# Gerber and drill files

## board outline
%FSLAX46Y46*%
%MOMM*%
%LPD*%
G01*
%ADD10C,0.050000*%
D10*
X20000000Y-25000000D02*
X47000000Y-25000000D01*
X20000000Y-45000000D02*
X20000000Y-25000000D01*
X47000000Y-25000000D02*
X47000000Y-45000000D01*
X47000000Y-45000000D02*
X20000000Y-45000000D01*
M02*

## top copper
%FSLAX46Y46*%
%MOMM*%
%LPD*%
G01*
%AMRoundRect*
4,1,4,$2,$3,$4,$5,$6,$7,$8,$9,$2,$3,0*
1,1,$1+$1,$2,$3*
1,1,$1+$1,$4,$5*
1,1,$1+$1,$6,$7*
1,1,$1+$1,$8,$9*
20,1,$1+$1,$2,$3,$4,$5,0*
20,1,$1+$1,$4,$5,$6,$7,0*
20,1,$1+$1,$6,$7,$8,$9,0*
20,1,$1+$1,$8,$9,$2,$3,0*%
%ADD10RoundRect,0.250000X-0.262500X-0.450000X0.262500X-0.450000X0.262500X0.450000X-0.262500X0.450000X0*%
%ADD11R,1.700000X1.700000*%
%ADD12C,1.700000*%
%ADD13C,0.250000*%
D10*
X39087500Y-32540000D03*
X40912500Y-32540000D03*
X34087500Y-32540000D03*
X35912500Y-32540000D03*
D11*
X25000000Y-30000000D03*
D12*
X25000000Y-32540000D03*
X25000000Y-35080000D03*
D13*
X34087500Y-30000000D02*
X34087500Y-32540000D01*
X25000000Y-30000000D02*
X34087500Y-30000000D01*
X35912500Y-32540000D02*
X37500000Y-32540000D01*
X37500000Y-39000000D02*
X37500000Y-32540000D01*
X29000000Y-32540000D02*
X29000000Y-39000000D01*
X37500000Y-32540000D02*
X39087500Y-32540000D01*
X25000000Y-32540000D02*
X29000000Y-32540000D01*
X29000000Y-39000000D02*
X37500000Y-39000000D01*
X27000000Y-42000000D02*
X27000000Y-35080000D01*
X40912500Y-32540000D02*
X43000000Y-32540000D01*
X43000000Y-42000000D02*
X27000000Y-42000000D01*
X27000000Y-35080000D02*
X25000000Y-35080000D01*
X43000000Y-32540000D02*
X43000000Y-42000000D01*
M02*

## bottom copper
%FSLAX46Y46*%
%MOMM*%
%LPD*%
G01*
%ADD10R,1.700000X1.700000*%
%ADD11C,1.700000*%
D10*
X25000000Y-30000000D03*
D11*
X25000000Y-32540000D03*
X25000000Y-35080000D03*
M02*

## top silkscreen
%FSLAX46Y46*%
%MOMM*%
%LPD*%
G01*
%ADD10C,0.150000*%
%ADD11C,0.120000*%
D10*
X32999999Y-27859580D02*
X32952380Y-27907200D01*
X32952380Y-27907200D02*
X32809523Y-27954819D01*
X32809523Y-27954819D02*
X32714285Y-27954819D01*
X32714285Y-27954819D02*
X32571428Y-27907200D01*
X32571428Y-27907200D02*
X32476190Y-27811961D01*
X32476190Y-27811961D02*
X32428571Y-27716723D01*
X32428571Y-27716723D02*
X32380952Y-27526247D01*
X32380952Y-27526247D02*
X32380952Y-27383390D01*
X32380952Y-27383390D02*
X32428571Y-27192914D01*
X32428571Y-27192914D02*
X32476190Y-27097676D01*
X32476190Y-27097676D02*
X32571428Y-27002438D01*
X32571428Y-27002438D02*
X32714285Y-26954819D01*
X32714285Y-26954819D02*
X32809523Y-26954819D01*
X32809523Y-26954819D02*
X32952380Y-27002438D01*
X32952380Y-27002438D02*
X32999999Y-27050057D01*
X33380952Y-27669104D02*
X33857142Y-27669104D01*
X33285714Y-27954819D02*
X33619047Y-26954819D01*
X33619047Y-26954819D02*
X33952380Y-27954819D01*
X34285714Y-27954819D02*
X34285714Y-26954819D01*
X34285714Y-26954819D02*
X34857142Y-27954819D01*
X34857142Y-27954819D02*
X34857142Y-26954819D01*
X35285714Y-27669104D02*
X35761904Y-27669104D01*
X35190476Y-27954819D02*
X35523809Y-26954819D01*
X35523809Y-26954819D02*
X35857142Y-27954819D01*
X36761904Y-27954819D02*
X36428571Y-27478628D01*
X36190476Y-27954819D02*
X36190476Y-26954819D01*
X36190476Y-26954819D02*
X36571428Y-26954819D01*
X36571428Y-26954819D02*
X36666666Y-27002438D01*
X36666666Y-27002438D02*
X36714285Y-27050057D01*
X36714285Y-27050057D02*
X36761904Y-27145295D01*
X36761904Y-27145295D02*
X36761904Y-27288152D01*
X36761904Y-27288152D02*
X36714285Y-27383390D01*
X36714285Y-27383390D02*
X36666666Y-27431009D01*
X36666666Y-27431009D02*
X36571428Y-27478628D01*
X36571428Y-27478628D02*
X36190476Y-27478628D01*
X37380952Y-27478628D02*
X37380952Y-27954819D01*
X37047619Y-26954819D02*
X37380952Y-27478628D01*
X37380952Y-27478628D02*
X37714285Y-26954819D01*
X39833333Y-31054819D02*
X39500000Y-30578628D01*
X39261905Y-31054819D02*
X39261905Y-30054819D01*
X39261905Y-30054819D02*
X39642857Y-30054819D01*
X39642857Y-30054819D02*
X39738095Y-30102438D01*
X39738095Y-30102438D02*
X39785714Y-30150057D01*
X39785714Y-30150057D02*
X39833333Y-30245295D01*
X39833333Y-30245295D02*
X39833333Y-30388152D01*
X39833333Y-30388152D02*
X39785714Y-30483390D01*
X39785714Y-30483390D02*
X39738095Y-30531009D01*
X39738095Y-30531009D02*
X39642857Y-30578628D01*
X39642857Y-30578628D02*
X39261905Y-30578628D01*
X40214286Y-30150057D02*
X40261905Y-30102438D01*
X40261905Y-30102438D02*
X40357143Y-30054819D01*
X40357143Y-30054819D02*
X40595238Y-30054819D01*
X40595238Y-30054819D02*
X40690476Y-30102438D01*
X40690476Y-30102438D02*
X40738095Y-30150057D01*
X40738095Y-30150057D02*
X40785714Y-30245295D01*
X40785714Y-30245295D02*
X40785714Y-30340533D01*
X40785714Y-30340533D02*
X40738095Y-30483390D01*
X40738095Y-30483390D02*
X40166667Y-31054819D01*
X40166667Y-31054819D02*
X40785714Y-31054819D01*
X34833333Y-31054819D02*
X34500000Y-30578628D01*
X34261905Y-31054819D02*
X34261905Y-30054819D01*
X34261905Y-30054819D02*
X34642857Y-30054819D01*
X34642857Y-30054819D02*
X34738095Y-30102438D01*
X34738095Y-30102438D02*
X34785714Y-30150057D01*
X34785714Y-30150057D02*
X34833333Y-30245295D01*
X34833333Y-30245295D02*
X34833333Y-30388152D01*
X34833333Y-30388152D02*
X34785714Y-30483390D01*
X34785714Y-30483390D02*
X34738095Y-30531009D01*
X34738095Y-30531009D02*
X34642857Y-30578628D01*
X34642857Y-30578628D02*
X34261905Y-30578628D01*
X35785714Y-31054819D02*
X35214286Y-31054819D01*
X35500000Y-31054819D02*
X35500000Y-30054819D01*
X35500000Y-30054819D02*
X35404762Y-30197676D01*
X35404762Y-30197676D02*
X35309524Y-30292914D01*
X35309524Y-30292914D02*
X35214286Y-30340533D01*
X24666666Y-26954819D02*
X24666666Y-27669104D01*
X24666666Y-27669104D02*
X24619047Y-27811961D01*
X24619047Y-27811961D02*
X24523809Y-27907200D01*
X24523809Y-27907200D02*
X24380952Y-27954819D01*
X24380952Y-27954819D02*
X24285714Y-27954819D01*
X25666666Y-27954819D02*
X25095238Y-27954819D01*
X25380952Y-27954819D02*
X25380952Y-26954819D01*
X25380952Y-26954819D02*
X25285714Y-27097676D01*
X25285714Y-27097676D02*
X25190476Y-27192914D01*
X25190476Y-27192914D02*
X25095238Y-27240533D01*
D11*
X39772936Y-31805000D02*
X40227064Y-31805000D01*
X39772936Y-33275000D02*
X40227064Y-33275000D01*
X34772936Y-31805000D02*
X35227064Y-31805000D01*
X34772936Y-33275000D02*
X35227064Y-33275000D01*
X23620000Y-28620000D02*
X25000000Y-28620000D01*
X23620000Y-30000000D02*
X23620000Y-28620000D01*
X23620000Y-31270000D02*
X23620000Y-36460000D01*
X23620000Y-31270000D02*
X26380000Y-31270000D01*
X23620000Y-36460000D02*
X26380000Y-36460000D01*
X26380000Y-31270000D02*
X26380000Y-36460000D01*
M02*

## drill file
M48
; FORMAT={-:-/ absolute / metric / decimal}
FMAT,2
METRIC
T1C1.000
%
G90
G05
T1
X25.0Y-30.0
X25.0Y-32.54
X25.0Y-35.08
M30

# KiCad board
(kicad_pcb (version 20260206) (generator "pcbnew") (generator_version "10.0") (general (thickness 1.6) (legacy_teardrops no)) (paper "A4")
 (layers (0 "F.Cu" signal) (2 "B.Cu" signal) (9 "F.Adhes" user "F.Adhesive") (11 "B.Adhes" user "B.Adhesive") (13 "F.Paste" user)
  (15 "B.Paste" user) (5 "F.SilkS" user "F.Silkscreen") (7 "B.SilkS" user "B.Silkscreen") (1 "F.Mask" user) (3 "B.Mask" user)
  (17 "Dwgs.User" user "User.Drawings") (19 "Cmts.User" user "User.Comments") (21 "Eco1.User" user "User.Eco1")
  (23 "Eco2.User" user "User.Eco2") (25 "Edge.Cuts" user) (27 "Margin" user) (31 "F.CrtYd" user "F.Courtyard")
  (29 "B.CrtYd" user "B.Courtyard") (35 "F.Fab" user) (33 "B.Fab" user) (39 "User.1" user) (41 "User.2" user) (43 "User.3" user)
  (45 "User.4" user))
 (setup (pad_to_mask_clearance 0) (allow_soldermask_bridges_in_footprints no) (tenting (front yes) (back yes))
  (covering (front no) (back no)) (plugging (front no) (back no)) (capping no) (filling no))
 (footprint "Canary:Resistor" (layer "F.Cu") (at 40 32.54)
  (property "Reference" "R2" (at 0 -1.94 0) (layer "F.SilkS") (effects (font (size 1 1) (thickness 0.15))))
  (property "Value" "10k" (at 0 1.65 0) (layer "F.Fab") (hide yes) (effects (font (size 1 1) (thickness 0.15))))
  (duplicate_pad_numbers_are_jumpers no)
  (fp_line (start -0.227064 -0.735) (end 0.227064 -0.735) (stroke (width 0.12) (type solid)) (layer "F.SilkS"))
  (fp_line (start -0.227064 0.735) (end 0.227064 0.735) (stroke (width 0.12) (type solid)) (layer "F.SilkS"))
  (pad "1" smd roundrect (at -0.9125 0) (size 1.025 1.4) (layers "F.Cu" "F.Mask" "F.Paste") (roundrect_rratio 0.243902) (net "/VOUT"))
  (pad "2" smd roundrect (at 0.9125 0) (size 1.025 1.4) (layers "F.Cu" "F.Mask" "F.Paste") (roundrect_rratio 0.243902) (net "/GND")))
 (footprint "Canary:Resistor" (layer "F.Cu") (at 35 32.54)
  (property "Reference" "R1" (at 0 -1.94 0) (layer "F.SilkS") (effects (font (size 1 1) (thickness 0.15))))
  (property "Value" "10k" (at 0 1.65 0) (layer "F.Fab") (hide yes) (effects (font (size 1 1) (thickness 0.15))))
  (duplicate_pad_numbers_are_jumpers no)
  (fp_line (start -0.227064 -0.735) (end 0.227064 -0.735) (stroke (width 0.12) (type solid)) (layer "F.SilkS"))
  (fp_line (start -0.227064 0.735) (end 0.227064 0.735) (stroke (width 0.12) (type solid)) (layer "F.SilkS"))
  (pad "1" smd roundrect (at -0.9125 0) (size 1.025 1.4) (layers "F.Cu" "F.Mask" "F.Paste") (roundrect_rratio 0.243902) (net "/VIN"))
  (pad "2" smd roundrect (at 0.9125 0) (size 1.025 1.4) (layers "F.Cu" "F.Mask" "F.Paste") (roundrect_rratio 0.243902) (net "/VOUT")))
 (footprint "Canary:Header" (layer "F.Cu") (at 25 30)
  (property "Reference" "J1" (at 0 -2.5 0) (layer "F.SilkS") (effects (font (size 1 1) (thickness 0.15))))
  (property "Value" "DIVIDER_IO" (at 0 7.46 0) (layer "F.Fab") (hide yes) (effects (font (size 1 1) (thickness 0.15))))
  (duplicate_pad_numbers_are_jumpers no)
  (fp_line (start -1.38 -1.38) (end 0 -1.38) (stroke (width 0.12) (type solid)) (layer "F.SilkS"))
  (fp_line (start -1.38 0) (end -1.38 -1.38) (stroke (width 0.12) (type solid)) (layer "F.SilkS"))
  (fp_line (start -1.38 1.27) (end -1.38 6.46) (stroke (width 0.12) (type solid)) (layer "F.SilkS"))
  (fp_line (start -1.38 1.27) (end 1.38 1.27) (stroke (width 0.12) (type solid)) (layer "F.SilkS"))
  (fp_line (start -1.38 6.46) (end 1.38 6.46) (stroke (width 0.12) (type solid)) (layer "F.SilkS"))
  (fp_line (start 1.38 1.27) (end 1.38 6.46) (stroke (width 0.12) (type solid)) (layer "F.SilkS"))
  (pad "1" thru_hole rect (at 0 0) (size 1.7 1.7) (drill 1) (layers "*.Cu" "*.Mask") (remove_unused_layers no) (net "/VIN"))
  (pad "2" thru_hole circle (at 0 2.54) (size 1.7 1.7) (drill 1) (layers "*.Cu" "*.Mask") (remove_unused_layers no) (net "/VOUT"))
  (pad "3" thru_hole circle (at 0 5.08) (size 1.7 1.7) (drill 1) (layers "*.Cu" "*.Mask") (remove_unused_layers no) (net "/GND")))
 (gr_line (start 20 25) (end 47 25) (stroke (width 0.05) (type default)) (layer "Edge.Cuts"))
 (gr_line (start 20 45) (end 20 25) (stroke (width 0.05) (type default)) (layer "Edge.Cuts"))
 (gr_line (start 47 25) (end 47 45) (stroke (width 0.05) (type default)) (layer "Edge.Cuts"))
 (gr_line (start 47 45) (end 20 45) (stroke (width 0.05) (type default)) (layer "Edge.Cuts"))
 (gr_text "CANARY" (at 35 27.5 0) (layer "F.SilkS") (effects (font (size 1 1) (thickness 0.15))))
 (segment (start 34.0875 30) (end 34.0875 32.54) (width 0.25) (layer "F.Cu") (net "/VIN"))
 (segment (start 25 30) (end 34.0875 30) (width 0.25) (layer "F.Cu") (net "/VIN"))
 (segment (start 35.9125 32.54) (end 37.5 32.54) (width 0.25) (layer "F.Cu") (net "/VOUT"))
 (segment (start 37.5 39) (end 37.5 32.54) (width 0.25) (layer "F.Cu") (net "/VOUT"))
 (segment (start 29 32.54) (end 29 39) (width 0.25) (layer "F.Cu") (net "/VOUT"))
 (segment (start 37.5 32.54) (end 39.0875 32.54) (width 0.25) (layer "F.Cu") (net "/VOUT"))
 (segment (start 25 32.54) (end 29 32.54) (width 0.25) (layer "F.Cu") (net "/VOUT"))
 (segment (start 29 39) (end 37.5 39) (width 0.25) (layer "F.Cu") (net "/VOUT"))
 (segment (start 27 42) (end 27 35.08) (width 0.25) (layer "F.Cu") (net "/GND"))
 (segment (start 40.9125 32.54) (end 43 32.54) (width 0.25) (layer "F.Cu") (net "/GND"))
 (segment (start 43 42) (end 27 42) (width 0.25) (layer "F.Cu") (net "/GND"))
 (segment (start 27 35.08) (end 25 35.08) (width 0.25) (layer "F.Cu") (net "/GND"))
 (segment (start 43 32.54) (end 43 42) (width 0.25) (layer "F.Cu") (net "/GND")))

